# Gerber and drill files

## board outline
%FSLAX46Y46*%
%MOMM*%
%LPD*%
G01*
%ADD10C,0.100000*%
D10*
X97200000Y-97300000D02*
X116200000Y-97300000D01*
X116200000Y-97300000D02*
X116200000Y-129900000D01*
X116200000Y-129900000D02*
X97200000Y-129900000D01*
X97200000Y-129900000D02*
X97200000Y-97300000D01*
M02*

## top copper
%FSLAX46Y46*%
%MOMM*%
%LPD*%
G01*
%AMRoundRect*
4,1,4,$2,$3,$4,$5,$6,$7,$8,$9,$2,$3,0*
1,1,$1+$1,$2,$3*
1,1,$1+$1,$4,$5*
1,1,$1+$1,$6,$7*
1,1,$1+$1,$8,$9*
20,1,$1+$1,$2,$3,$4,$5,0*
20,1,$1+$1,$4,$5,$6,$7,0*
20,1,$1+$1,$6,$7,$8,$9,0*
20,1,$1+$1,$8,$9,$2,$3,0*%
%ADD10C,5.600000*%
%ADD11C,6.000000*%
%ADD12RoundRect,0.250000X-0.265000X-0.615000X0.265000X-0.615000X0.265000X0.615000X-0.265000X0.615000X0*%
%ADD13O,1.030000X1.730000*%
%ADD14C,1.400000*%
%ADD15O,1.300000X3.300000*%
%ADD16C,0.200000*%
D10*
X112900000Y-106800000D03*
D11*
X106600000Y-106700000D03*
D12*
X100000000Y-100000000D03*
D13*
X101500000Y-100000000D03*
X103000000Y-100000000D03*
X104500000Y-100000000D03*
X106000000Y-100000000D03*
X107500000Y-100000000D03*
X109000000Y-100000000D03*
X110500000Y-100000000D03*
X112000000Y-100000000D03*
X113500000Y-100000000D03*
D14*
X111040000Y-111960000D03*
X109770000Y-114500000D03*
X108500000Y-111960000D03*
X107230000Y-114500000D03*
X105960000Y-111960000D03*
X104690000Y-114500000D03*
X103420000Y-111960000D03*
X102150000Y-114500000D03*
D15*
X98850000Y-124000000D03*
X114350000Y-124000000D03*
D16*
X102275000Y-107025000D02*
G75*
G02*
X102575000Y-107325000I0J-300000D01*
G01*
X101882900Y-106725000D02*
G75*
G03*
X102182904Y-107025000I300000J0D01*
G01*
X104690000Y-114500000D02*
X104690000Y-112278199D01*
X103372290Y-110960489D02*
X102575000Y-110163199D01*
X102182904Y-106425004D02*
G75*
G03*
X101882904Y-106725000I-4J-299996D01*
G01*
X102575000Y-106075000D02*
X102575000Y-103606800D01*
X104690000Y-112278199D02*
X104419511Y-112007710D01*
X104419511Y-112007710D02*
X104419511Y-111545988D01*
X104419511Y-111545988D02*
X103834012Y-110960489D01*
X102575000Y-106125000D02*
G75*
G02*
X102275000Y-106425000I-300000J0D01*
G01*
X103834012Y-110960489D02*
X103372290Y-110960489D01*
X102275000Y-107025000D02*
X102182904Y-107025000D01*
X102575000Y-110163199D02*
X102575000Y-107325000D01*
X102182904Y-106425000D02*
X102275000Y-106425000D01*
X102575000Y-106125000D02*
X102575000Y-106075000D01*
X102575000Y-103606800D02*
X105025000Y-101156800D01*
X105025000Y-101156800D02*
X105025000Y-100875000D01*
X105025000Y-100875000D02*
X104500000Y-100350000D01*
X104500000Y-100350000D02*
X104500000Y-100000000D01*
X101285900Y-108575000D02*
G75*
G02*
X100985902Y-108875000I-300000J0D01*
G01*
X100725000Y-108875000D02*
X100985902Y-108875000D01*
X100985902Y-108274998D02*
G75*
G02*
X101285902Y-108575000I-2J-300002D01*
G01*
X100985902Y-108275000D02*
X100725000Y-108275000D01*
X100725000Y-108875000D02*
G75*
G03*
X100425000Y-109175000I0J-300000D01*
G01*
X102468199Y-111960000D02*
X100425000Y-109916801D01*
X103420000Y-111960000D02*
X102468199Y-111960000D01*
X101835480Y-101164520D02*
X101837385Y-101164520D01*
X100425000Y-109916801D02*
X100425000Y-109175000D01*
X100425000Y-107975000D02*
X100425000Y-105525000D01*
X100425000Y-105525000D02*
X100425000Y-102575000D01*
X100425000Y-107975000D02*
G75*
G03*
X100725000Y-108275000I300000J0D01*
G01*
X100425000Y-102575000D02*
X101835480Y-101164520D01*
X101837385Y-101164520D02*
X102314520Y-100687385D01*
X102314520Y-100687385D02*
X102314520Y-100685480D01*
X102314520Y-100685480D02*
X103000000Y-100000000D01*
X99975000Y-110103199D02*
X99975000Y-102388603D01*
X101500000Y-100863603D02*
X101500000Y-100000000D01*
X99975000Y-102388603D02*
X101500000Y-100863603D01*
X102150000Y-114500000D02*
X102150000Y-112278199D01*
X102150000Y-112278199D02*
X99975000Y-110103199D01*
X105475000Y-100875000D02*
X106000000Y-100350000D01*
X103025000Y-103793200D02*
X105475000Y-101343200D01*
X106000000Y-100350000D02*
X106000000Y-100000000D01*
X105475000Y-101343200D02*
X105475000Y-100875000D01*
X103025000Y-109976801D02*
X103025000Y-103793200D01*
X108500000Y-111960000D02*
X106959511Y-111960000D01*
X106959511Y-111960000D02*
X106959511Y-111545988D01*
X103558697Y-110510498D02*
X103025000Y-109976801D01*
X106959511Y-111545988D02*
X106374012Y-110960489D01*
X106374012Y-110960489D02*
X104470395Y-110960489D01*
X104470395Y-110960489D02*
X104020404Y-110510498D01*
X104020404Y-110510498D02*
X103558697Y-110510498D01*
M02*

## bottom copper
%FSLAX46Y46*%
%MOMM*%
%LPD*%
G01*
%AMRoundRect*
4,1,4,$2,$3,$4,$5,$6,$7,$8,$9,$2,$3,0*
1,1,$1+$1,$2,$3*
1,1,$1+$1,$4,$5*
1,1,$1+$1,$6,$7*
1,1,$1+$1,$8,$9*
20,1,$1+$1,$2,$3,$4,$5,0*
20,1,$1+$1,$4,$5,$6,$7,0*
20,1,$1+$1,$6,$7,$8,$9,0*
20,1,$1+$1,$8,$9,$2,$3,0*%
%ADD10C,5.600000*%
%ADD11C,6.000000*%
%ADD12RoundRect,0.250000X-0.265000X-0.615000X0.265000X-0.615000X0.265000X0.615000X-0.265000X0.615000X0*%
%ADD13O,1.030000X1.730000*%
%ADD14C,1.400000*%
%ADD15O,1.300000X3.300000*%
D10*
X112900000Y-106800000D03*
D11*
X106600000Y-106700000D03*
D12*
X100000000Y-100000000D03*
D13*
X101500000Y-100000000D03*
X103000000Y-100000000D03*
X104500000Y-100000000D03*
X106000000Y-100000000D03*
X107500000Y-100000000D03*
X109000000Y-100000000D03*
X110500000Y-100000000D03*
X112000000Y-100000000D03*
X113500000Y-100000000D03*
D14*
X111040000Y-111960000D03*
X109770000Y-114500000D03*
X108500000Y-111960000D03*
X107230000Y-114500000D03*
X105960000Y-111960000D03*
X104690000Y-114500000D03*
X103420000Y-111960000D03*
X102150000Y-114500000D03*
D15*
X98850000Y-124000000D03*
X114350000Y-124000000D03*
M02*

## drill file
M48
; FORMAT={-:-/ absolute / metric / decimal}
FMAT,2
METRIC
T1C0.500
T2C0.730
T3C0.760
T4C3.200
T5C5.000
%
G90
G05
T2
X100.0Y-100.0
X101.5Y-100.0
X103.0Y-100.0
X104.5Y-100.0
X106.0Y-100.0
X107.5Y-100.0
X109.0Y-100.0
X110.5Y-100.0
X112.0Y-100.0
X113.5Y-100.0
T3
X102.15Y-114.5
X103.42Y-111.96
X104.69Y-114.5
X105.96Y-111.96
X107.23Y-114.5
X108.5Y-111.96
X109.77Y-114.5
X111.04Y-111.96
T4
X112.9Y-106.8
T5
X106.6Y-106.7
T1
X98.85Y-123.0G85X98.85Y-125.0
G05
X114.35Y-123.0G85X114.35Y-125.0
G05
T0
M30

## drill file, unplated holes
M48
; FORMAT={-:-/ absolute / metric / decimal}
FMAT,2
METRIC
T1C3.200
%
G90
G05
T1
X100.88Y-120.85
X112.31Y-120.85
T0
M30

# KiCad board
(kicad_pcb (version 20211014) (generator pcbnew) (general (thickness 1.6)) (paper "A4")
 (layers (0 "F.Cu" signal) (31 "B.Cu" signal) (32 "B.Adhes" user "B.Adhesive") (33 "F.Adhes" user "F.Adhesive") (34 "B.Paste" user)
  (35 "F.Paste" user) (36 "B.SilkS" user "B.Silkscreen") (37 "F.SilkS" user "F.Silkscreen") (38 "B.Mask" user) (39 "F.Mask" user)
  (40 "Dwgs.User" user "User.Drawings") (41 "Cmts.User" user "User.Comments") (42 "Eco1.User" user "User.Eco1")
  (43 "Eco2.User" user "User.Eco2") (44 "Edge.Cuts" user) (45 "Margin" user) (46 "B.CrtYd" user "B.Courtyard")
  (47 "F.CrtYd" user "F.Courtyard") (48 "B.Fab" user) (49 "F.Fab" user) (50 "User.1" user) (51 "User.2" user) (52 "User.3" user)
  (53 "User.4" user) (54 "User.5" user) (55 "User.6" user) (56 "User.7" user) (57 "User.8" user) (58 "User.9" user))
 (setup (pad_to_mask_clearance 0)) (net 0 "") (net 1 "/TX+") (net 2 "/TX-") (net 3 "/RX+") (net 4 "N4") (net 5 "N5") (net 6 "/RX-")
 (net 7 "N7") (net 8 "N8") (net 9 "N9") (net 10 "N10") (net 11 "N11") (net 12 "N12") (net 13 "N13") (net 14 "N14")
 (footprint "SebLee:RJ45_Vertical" (layer "F.Cu") (at 102.15 114.5)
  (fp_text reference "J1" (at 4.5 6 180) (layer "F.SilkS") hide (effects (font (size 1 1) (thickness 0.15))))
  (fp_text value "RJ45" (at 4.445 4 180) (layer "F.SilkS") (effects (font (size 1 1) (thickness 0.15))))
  (pad "" np_thru_hole circle locked (at -1.27 6.35) (size 3.2 3.2) (drill 3.2) (layers *.Cu *.Mask))
  (pad "" np_thru_hole circle locked (at 10.16 6.35) (size 3.2 3.2) (drill 3.2) (layers *.Cu *.Mask))
  (pad "1" thru_hole circle locked (at 0 0) (size 1.4 1.4) (drill 0.76) (layers *.Cu *.Mask) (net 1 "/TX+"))
  (pad "2" thru_hole circle locked (at 1.27 -2.54) (size 1.4 1.4) (drill 0.76) (layers *.Cu *.Mask) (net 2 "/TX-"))
  (pad "3" thru_hole circle locked (at 2.54 0) (size 1.4 1.4) (drill 0.76) (layers *.Cu *.Mask) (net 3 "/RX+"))
  (pad "4" thru_hole circle locked (at 3.81 -2.54) (size 1.4 1.4) (drill 0.76) (layers *.Cu *.Mask) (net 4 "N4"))
  (pad "5" thru_hole circle locked (at 5.08 0) (size 1.4 1.4) (drill 0.76) (layers *.Cu *.Mask) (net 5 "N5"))
  (pad "6" thru_hole circle locked (at 6.35 -2.54) (size 1.4 1.4) (drill 0.76) (layers *.Cu *.Mask) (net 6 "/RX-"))
  (pad "7" thru_hole circle locked (at 7.62 0) (size 1.4 1.4) (drill 0.76) (layers *.Cu *.Mask) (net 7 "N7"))
  (pad "8" thru_hole circle locked (at 8.89 -2.54) (size 1.4 1.4) (drill 0.76) (layers *.Cu *.Mask) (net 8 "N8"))
  (pad "SH" thru_hole oval locked (at -3.3 9.5) (size 1.3 3.3) (drill oval 0.5 2.5) (layers *.Cu *.Mask))
  (pad "SH" thru_hole oval locked (at 12.2 9.5) (size 1.3 3.3) (drill oval 0.5 2.5) (layers *.Cu *.Mask)))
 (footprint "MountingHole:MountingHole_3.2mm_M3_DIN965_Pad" (layer "F.Cu") (at 112.9 106.8)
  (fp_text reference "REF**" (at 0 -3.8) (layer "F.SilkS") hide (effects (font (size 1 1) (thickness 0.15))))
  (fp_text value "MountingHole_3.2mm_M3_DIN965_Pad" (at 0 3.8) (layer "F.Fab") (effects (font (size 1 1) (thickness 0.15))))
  (pad "1" thru_hole circle (at 0 0) (size 5.6 5.6) (drill 3.2) (layers *.Cu *.Mask)))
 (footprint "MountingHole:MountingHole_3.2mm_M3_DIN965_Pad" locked (layer "F.Cu") (at 106.6 106.7)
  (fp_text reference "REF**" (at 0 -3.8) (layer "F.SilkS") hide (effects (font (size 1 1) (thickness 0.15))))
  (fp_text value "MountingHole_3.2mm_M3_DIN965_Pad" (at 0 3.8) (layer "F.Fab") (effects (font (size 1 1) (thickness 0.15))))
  (pad "1" thru_hole circle locked (at 0 0) (size 6 6) (drill 5) (layers *.Cu *.Mask)))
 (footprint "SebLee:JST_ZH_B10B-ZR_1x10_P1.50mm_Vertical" (layer "F.Cu") (at 100 100)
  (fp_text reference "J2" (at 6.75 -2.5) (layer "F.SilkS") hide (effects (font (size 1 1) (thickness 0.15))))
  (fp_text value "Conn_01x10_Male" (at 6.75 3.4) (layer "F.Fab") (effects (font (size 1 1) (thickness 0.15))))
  (pad "1" thru_hole roundrect locked (at 0 0) (size 1.03 1.73) (drill 0.73) (layers *.Cu *.Mask) (roundrect_rratio 0.2427184466)
   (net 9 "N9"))
  (pad "2" thru_hole oval locked (at 1.5 0) (size 1.03 1.73) (drill 0.73) (layers *.Cu *.Mask) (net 1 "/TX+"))
  (pad "3" thru_hole oval locked (at 3 0) (size 1.03 1.73) (drill 0.73) (layers *.Cu *.Mask) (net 2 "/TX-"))
  (pad "4" thru_hole oval locked (at 4.5 0) (size 1.03 1.73) (drill 0.73) (layers *.Cu *.Mask) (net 3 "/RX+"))
  (pad "5" thru_hole oval locked (at 6 0) (size 1.03 1.73) (drill 0.73) (layers *.Cu *.Mask) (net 6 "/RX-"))
  (pad "6" thru_hole oval locked (at 7.5 0) (size 1.03 1.73) (drill 0.73) (layers *.Cu *.Mask) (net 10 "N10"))
  (pad "7" thru_hole oval locked (at 9 0) (size 1.03 1.73) (drill 0.73) (layers *.Cu *.Mask) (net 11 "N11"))
  (pad "8" thru_hole oval locked (at 10.5 0) (size 1.03 1.73) (drill 0.73) (layers *.Cu *.Mask) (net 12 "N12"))
  (pad "9" thru_hole oval locked (at 12 0) (size 1.03 1.73) (drill 0.73) (layers *.Cu *.Mask) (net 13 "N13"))
  (pad "10" thru_hole oval locked (at 13.5 0) (size 1.03 1.73) (drill 0.73) (layers *.Cu *.Mask) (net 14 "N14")))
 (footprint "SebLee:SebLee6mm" (layer "B.Cu") (at 106.7 120.3 180)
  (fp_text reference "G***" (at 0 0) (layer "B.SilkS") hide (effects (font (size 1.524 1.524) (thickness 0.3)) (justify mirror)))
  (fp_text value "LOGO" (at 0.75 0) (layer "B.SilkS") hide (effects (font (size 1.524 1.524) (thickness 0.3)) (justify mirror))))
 (gr_rect (start 97.2 97.3) (end 116.2 129.9) (layer "Edge.Cuts") (width 0.1) (fill none))
 (segment (start 106.959511 111.96) (end 106.959511 111.545988) (width 0.2) (layer "F.Cu") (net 6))
 (segment (start 105.475 101.3432) (end 105.475 100.875) (width 0.2) (layer "F.Cu") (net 6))
 (segment (start 106.374012 110.960489) (end 104.470395 110.960489) (width 0.2) (layer "F.Cu") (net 6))
 (segment (start 108.5 111.96) (end 106.959511 111.96) (width 0.2) (layer "F.Cu") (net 6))
 (segment (start 103.025 109.976801) (end 103.025 103.7932) (width 0.2) (layer "F.Cu") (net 6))
 (segment (start 103.558697 110.510498) (end 103.025 109.976801) (width 0.2) (layer "F.Cu") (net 6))
 (segment (start 106 100.35) (end 106 100) (width 0.2) (layer "F.Cu") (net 6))
 (segment (start 105.475 100.875) (end 106 100.35) (width 0.2) (layer "F.Cu") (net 6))
 (segment (start 104.020404 110.510498) (end 103.558697 110.510498) (width 0.2) (layer "F.Cu") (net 6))
 (segment (start 104.470395 110.960489) (end 104.020404 110.510498) (width 0.2) (layer "F.Cu") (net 6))
 (segment (start 103.025 103.7932) (end 105.475 101.3432) (width 0.2) (layer "F.Cu") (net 6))
 (segment (start 106.959511 111.545988) (end 106.374012 110.960489) (width 0.2) (layer "F.Cu") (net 6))
 (segment (start 104.419511 112.00771) (end 104.419511 111.545988) (width 0.2) (layer "F.Cu") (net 3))
 (segment (start 104.69 112.278199) (end 104.419511 112.00771) (width 0.2) (layer "F.Cu") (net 3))
 (segment (start 102.182904 106.425) (end 102.275 106.425) (width 0.2) (layer "F.Cu") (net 3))
 (segment (start 102.575 106.075) (end 102.575 103.6068) (width 0.2) (layer "F.Cu") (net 3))
 (segment (start 103.834012 110.960489) (end 103.37229 110.960489) (width 0.2) (layer "F.Cu") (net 3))
 (segment (start 102.575 110.163199) (end 102.575 107.325) (width 0.2) (layer "F.Cu") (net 3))
 (segment (start 102.275 107.025) (end 102.182904 107.025) (width 0.2) (layer "F.Cu") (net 3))
 (segment (start 104.419511 111.545988) (end 103.834012 110.960489) (width 0.2) (layer "F.Cu") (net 3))
 (segment (start 104.5 100.35) (end 104.5 100) (width 0.2) (layer "F.Cu") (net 3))
 (segment (start 102.575 106.125) (end 102.575 106.075) (width 0.2) (layer "F.Cu") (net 3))
 (segment (start 102.575 103.6068) (end 105.025 101.1568) (width 0.2) (layer "F.Cu") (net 3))
 (segment (start 104.69 114.5) (end 104.69 112.278199) (width 0.2) (layer "F.Cu") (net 3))
 (segment (start 105.025 101.1568) (end 105.025 100.875) (width 0.2) (layer "F.Cu") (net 3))
 (segment (start 103.37229 110.960489) (end 102.575 110.163199) (width 0.2) (layer "F.Cu") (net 3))
 (segment (start 105.025 100.875) (end 104.5 100.35) (width 0.2) (layer "F.Cu") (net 3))
 (arc (start 102.182904 107.025) (mid 101.970772 106.937132) (end 101.882904 106.725) (width 0.2) (layer "F.Cu") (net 3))
 (arc (start 102.575 107.325) (mid 102.487132 107.112868) (end 102.275 107.025) (width 0.2) (layer "F.Cu") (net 3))
 (arc (start 101.882904 106.725) (mid 101.970772 106.512868) (end 102.182904 106.425) (width 0.2) (layer "F.Cu") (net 3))
 (arc (start 102.275 106.425) (mid 102.487132 106.337132) (end 102.575 106.125) (width 0.2) (layer "F.Cu") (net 3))
 (segment (start 102.31452 100.687385) (end 102.31452 100.68548) (width 0.2) (layer "F.Cu") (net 2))
 (segment (start 100.985902 108.275) (end 100.725 108.275) (width 0.2) (layer "F.Cu") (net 2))
 (segment (start 100.425 109.916801) (end 100.425 109.175) (width 0.2) (layer "F.Cu") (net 2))
 (segment (start 101.837385 101.16452) (end 102.31452 100.687385) (width 0.2) (layer "F.Cu") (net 2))
 (segment (start 100.425 102.575) (end 101.83548 101.16452) (width 0.2) (layer "F.Cu") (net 2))
 (segment (start 100.425 105.525) (end 100.425 102.575) (width 0.2) (layer "F.Cu") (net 2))
 (segment (start 100.425 107.975) (end 100.425 105.525) (width 0.2) (layer "F.Cu") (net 2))
 (segment (start 102.468199 111.96) (end 100.425 109.916801) (width 0.2) (layer "F.Cu") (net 2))
 (segment (start 101.83548 101.16452) (end 101.837385 101.16452) (width 0.2) (layer "F.Cu") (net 2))
 (segment (start 100.725 108.875) (end 100.985902 108.875) (width 0.2) (layer "F.Cu") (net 2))
 (segment (start 103.42 111.96) (end 102.468199 111.96) (width 0.2) (layer "F.Cu") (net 2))
 (segment (start 102.31452 100.68548) (end 103 100) (width 0.2) (layer "F.Cu") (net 2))
 (arc (start 101.285902 108.575) (mid 101.198034 108.362868) (end 100.985902 108.275) (width 0.2) (layer "F.Cu") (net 2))
 (arc (start 100.425 109.175) (mid 100.512868 108.962868) (end 100.725 108.875) (width 0.2) (layer "F.Cu") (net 2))
 (arc (start 100.985902 108.875) (mid 101.198034 108.787132) (end 101.285902 108.575) (width 0.2) (layer "F.Cu") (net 2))
 (arc (start 100.725 108.275) (mid 100.512868 108.187132) (end 100.425 107.975) (width 0.2) (layer "F.Cu") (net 2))
 (segment (start 99.975 110.103199) (end 99.975 102.388603) (width 0.2) (layer "F.Cu") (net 1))
 (segment (start 102.15 112.278199) (end 99.975 110.103199) (width 0.2) (layer "F.Cu") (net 1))
 (segment (start 101.5 100.863603) (end 101.5 100) (width 0.2) (layer "F.Cu") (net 1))
 (segment (start 102.15 114.5) (end 102.15 112.278199) (width 0.2) (layer "F.Cu") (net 1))
 (segment (start 99.975 102.388603) (end 101.5 100.863603) (width 0.2) (layer "F.Cu") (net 1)))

